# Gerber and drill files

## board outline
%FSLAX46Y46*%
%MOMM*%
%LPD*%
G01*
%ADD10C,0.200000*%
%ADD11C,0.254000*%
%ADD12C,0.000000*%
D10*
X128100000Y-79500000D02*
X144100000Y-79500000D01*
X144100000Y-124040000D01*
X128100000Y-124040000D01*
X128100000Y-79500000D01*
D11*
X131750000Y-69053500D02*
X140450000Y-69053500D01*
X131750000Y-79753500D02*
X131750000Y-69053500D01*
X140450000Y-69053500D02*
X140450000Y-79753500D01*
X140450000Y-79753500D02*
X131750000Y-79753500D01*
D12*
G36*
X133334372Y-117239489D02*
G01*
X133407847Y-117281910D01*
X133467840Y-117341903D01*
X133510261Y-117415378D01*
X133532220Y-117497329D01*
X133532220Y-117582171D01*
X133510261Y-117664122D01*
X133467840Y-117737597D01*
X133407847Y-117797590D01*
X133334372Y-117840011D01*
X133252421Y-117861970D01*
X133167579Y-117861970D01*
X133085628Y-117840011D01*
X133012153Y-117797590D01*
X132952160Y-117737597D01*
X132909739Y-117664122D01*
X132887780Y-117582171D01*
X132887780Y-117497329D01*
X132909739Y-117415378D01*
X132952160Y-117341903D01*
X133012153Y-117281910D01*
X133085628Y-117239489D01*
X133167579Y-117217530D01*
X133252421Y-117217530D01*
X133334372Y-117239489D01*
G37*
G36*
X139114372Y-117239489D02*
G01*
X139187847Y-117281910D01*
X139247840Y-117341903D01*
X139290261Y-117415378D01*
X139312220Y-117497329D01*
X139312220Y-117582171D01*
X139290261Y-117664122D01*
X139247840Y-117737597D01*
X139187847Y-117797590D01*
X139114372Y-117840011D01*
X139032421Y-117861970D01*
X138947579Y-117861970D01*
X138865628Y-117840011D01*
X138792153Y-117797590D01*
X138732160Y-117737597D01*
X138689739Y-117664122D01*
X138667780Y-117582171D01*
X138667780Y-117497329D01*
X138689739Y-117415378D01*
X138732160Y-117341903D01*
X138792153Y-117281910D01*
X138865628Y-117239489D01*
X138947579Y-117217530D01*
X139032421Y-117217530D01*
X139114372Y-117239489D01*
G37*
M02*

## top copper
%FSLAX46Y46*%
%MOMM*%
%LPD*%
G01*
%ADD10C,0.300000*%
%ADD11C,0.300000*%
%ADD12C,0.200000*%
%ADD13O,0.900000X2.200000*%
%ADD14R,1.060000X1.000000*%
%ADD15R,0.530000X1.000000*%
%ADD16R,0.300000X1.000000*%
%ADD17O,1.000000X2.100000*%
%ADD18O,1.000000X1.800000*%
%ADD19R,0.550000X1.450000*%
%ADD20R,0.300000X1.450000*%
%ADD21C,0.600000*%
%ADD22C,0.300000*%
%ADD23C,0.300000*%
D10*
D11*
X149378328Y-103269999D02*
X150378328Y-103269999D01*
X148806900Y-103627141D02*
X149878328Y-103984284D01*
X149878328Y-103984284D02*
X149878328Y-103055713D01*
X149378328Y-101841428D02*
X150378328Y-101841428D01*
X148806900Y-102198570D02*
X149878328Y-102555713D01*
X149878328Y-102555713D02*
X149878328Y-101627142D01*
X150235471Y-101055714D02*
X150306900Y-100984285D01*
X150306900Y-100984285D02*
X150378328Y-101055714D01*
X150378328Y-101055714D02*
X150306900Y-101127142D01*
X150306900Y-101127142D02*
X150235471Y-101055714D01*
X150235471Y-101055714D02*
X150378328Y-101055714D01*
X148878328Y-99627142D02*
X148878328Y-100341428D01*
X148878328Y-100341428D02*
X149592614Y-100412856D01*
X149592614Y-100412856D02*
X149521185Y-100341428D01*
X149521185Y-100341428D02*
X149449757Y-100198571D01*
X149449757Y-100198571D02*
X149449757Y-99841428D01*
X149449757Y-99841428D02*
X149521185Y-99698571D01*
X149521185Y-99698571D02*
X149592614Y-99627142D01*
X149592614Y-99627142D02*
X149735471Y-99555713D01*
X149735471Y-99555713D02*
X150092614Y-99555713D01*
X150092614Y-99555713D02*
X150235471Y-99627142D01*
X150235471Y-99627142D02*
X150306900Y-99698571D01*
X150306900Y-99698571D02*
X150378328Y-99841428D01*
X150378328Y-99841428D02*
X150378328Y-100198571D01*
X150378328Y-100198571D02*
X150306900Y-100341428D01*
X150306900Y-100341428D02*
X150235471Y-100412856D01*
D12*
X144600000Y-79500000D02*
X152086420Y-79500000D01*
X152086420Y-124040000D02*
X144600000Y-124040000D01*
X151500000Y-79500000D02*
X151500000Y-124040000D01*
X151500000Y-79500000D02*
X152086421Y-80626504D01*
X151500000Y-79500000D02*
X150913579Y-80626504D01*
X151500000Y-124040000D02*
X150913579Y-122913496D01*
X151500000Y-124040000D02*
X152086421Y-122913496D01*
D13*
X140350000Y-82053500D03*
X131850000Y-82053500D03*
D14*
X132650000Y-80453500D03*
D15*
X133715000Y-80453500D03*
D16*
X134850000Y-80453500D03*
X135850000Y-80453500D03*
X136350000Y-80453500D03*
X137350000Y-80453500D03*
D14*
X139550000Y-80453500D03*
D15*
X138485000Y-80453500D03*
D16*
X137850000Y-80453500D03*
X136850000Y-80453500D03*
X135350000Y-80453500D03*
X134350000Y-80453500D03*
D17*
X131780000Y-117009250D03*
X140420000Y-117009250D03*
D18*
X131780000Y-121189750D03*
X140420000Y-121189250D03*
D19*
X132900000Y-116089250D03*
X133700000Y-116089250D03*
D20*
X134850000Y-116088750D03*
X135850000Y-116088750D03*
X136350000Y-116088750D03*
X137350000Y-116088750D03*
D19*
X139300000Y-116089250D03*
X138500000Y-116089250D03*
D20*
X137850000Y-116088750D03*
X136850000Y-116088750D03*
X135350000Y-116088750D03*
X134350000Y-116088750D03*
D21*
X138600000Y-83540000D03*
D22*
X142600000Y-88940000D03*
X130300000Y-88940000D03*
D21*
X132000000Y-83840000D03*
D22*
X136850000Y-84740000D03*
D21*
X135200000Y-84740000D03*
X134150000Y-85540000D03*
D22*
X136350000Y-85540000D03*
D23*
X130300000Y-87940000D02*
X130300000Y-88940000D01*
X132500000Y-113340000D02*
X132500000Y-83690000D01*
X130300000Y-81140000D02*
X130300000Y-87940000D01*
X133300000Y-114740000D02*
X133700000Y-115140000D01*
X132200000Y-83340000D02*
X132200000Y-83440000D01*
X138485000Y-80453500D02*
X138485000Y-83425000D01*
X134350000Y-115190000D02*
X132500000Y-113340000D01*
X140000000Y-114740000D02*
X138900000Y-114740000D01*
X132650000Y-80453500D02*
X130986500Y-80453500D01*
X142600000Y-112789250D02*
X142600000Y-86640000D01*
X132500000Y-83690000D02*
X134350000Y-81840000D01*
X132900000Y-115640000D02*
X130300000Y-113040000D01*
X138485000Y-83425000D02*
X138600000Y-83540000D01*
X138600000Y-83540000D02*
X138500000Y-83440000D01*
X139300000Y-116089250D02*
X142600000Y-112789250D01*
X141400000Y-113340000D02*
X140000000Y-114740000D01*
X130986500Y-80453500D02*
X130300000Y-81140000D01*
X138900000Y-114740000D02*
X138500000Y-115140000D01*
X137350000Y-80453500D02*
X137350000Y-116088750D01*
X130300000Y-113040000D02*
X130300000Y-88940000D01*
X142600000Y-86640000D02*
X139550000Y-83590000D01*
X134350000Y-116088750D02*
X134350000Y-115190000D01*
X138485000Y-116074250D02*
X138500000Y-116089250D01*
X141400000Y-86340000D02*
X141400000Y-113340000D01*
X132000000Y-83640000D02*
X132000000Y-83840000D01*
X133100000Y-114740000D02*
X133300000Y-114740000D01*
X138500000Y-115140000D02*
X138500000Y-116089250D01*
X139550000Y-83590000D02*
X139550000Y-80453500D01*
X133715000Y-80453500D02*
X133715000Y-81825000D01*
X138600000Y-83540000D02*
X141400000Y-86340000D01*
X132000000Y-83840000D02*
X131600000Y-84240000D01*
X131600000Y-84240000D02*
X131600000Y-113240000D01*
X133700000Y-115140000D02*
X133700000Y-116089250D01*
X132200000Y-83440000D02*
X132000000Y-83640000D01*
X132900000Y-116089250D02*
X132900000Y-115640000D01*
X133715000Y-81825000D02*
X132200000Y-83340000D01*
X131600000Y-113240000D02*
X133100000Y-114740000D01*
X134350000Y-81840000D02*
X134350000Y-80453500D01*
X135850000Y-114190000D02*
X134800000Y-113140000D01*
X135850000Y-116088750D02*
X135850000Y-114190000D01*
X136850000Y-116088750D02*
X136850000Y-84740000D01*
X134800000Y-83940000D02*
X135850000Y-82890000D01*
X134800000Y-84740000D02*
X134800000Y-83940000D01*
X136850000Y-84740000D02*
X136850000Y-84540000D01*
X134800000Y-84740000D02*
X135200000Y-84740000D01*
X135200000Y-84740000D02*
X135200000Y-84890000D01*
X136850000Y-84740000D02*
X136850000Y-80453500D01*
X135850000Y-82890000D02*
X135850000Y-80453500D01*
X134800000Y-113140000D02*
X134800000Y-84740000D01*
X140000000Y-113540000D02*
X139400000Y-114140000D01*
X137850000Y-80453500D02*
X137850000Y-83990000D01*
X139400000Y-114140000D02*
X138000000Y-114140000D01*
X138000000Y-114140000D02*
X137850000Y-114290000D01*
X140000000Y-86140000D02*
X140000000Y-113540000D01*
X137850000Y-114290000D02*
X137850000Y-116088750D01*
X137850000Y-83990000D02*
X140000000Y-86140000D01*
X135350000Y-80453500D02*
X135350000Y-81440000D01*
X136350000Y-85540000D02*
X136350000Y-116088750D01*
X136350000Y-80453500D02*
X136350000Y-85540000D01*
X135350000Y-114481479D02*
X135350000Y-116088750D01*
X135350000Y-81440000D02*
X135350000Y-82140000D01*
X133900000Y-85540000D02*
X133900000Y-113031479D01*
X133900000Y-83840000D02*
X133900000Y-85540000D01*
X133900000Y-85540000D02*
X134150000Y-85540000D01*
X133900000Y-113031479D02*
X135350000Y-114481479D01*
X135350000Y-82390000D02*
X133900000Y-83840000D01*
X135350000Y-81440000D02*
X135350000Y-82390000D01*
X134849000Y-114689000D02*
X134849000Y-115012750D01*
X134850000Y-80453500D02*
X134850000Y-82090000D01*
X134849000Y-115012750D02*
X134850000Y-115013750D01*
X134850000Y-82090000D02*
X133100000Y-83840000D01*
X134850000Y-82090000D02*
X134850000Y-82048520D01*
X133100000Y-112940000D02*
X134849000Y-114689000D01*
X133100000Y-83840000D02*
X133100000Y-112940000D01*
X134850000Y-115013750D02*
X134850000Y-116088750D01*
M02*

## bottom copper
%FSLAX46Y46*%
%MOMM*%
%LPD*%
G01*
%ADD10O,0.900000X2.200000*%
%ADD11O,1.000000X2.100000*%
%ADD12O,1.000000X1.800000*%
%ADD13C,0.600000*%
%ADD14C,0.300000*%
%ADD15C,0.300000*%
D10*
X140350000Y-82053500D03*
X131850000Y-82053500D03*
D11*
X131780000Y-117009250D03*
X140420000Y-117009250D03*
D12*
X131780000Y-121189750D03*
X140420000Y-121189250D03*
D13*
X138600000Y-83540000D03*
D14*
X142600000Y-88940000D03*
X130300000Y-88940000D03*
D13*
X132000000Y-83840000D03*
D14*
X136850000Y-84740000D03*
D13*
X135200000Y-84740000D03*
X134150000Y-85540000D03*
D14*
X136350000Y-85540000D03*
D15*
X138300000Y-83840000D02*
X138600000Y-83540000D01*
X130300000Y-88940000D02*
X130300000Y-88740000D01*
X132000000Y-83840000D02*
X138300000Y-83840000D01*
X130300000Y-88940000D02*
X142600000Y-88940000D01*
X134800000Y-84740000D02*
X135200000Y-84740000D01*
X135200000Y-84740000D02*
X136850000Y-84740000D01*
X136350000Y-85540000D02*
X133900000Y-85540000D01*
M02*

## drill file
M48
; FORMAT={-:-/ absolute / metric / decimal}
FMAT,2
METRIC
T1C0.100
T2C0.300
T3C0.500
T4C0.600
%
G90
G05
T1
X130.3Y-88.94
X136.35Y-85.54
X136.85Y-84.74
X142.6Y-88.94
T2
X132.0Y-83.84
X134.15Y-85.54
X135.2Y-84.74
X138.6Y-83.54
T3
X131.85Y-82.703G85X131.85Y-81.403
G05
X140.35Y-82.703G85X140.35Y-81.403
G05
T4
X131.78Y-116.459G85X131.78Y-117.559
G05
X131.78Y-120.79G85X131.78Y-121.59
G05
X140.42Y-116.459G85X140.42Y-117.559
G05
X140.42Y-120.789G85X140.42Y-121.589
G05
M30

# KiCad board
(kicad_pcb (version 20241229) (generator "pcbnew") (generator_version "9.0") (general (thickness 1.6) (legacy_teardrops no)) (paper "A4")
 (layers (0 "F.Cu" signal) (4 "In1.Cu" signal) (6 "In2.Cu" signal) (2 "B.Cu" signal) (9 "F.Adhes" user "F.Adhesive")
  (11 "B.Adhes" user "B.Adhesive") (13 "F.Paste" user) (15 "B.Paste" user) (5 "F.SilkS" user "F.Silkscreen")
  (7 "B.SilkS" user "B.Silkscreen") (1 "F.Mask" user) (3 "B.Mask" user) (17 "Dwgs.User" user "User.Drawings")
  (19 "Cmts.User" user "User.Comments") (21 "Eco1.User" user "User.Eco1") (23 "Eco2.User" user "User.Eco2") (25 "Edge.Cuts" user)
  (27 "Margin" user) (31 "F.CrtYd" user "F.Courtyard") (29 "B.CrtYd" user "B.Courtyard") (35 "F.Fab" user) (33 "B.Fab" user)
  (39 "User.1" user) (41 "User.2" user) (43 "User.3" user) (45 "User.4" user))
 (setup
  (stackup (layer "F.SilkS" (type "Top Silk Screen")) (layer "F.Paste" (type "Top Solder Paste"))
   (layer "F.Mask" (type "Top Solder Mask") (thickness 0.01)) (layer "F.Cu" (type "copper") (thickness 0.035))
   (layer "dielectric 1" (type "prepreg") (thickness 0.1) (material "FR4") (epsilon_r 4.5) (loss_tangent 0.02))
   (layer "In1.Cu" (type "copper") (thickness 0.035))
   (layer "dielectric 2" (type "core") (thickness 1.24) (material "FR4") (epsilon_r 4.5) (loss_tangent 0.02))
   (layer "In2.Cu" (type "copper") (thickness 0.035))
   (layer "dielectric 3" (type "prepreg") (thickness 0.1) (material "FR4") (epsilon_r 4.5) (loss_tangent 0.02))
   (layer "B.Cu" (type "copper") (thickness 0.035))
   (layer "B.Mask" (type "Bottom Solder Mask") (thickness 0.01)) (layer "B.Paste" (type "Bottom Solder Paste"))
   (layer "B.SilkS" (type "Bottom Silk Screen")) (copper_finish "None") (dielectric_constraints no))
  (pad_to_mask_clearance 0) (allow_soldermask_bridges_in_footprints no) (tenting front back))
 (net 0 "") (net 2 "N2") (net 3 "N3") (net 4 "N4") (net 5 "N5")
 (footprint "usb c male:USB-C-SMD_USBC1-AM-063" (layer "F.Cu") (at 136.1 81.2535 180)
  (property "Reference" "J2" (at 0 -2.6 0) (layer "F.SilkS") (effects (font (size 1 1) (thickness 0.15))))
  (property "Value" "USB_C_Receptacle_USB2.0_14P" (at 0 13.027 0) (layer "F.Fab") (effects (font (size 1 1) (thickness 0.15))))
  (fp_line (start 4.35 12.2) (end -4.35 12.2) (stroke (width 0.254) (type default)) (layer "Edge.Cuts") (net 1))
  (fp_line (start 4.35 1.5) (end 4.35 12.2) (stroke (width 0.254) (type default)) (layer "Edge.Cuts") (net 1))
  (fp_line (start -4.35 12.2) (end -4.35 1.5) (stroke (width 0.254) (type default)) (layer "Edge.Cuts") (net 1))
  (fp_line (start -4.35 1.5) (end 4.35 1.5) (stroke (width 0.254) (type default)) (layer "Edge.Cuts") (net 1))
  (pad "1" thru_hole oval (at -4.25 -0.8 180) (size 0.9 2.2) (drill oval 0.5 1.8) (layers "*.Cu" "*.Mask") (remove_unused_layers no))
  (pad "2" thru_hole oval (at 4.25 -0.8 180) (size 0.9 2.2) (drill oval 0.5 1.8) (layers "*.Cu" "*.Mask") (remove_unused_layers no))
  (pad "A1B12" smd rect (at 3.45 0.8) (size 1.06 1) (layers "F.Cu" "F.Mask" "F.Paste"))
  (pad "A4B9" smd rect (at 2.385 0.8) (size 0.53 1) (layers "F.Cu" "F.Mask" "F.Paste"))
  (pad "A5" smd rect (at 1.25 0.8) (size 0.3 1) (layers "F.Cu" "F.Mask" "F.Paste") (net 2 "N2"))
  (pad "A6" smd rect (at 0.25 0.8 180) (size 0.3 1) (layers "F.Cu" "F.Mask" "F.Paste") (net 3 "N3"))
  (pad "A7" smd rect (at -0.25 0.8) (size 0.3 1) (layers "F.Cu" "F.Mask" "F.Paste") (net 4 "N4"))
  (pad "A8" smd rect (at -1.25 0.8) (size 0.3 1) (layers "F.Cu" "F.Mask" "F.Paste"))
  (pad "B1A12" smd rect (at -3.45 0.8) (size 1.06 1) (layers "F.Cu" "F.Mask" "F.Paste"))
  (pad "B4A9" smd rect (at -2.385 0.8) (size 0.53 1) (layers "F.Cu" "F.Mask" "F.Paste"))
  (pad "B5" smd rect (at -1.75 0.8) (size 0.3 1) (layers "F.Cu" "F.Mask" "F.Paste") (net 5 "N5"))
  (pad "B6" smd rect (at -0.75 0.8 180) (size 0.3 1) (layers "F.Cu" "F.Mask" "F.Paste") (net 3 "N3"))
  (pad "B7" smd rect (at 0.75 0.8) (size 0.3 1) (layers "F.Cu" "F.Mask" "F.Paste") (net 4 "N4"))
  (pad "B8" smd rect (at 1.75 0.8) (size 0.3 1) (layers "F.Cu" "F.Mask" "F.Paste")))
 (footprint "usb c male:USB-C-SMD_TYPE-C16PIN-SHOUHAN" (layer "F.Cu") (at 136.1 118.63925)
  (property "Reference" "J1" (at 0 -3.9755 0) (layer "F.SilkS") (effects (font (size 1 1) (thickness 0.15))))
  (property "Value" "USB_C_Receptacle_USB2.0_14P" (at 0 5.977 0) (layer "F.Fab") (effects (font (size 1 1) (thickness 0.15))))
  (fp_poly
   (pts (xy -2.56778 -1.141921) (xy -2.589739 -1.223872) (xy -2.63216 -1.297347) (xy -2.692153 -1.35734) (xy -2.765628 -1.399761)
    (xy -2.847579 -1.42172) (xy -2.932421 -1.42172) (xy -3.014372 -1.399761) (xy -3.087847 -1.35734) (xy -3.14784 -1.297347)
    (xy -3.190261 -1.223872) (xy -3.21222 -1.141921) (xy -3.21222 -1.057079) (xy -3.190261 -0.975128) (xy -3.14784 -0.901653)
    (xy -3.087847 -0.84166) (xy -3.014372 -0.799239) (xy -2.932421 -0.77728) (xy -2.847579 -0.77728) (xy -2.765628 -0.799239)
    (xy -2.692153 -0.84166) (xy -2.63216 -0.901653) (xy -2.589739 -0.975128) (xy -2.56778 -1.057079))
   (stroke (width 0) (type default)) (fill yes) (layer "Edge.Cuts") (net 1))
  (fp_poly
   (pts (xy 3.21222 -1.141921) (xy 3.190261 -1.223872) (xy 3.14784 -1.297347) (xy 3.087847 -1.35734) (xy 3.014372 -1.399761)
    (xy 2.932421 -1.42172) (xy 2.847579 -1.42172) (xy 2.765628 -1.399761) (xy 2.692153 -1.35734) (xy 2.63216 -1.297347)
    (xy 2.589739 -1.223872) (xy 2.56778 -1.141921) (xy 2.56778 -1.057079) (xy 2.589739 -0.975128) (xy 2.63216 -0.901653)
    (xy 2.692153 -0.84166) (xy 2.765628 -0.799239) (xy 2.847579 -0.77728) (xy 2.932421 -0.77728) (xy 3.014372 -0.799239)
    (xy 3.087847 -0.84166) (xy 3.14784 -0.901653) (xy 3.190261 -0.975128) (xy 3.21222 -1.057079))
   (stroke (width 0) (type default)) (fill yes) (layer "Edge.Cuts") (net 1))
  (pad "1" thru_hole oval (at -4.32 -1.63) (size 1 2.1) (drill oval 0.6 1.7) (layers "*.Cu" "*.Mask") (remove_unused_layers no))
  (pad "2" thru_hole oval (at 4.32 -1.63) (size 1 2.1) (drill oval 0.6 1.7) (layers "*.Cu" "*.Mask") (remove_unused_layers no))
  (pad "3" thru_hole oval (at -4.32 2.5505) (size 1 1.8) (drill oval 0.6 1.4) (layers "*.Cu" "*.Mask") (remove_unused_layers no))
  (pad "4" thru_hole oval (at 4.32 2.55) (size 1 1.8) (drill oval 0.6 1.4) (layers "*.Cu" "*.Mask") (remove_unused_layers no))
  (pad "A1B12" smd rect (at -3.2 -2.55) (size 0.55 1.45) (layers "F.Cu" "F.Mask" "F.Paste"))
  (pad "A4B9" smd rect (at -2.4 -2.55) (size 0.55 1.45) (layers "F.Cu" "F.Mask" "F.Paste"))
  (pad "A5" smd rect (at -1.25 -2.5505) (size 0.3 1.45) (layers "F.Cu" "F.Mask" "F.Paste") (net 2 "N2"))
  (pad "A6" smd rect (at -0.25 -2.5505) (size 0.3 1.45) (layers "F.Cu" "F.Mask" "F.Paste") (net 3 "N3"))
  (pad "A7" smd rect (at 0.25 -2.5505) (size 0.3 1.45) (layers "F.Cu" "F.Mask" "F.Paste") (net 4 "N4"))
  (pad "A8" smd rect (at 1.25 -2.5505) (size 0.3 1.45) (layers "F.Cu" "F.Mask" "F.Paste"))
  (pad "B1A12" smd rect (at 3.2 -2.55) (size 0.55 1.45) (layers "F.Cu" "F.Mask" "F.Paste"))
  (pad "B4A9" smd rect (at 2.4 -2.55) (size 0.55 1.45) (layers "F.Cu" "F.Mask" "F.Paste"))
  (pad "B5" smd rect (at 1.75 -2.5505) (size 0.3 1.45) (layers "F.Cu" "F.Mask" "F.Paste") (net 5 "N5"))
  (pad "B6" smd rect (at 0.75 -2.5505) (size 0.3 1.45) (layers "F.Cu" "F.Mask" "F.Paste") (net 3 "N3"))
  (pad "B7" smd rect (at -0.75 -2.5505) (size 0.3 1.45) (layers "F.Cu" "F.Mask" "F.Paste") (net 4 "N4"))
  (pad "B8" smd rect (at -1.75 -2.5505) (size 0.3 1.45) (layers "F.Cu" "F.Mask" "F.Paste")))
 (gr_rect (start 128.1 79.5) (end 144.1 124.04) (stroke (width 0.2) (type solid)) (fill no) (layer "Edge.Cuts"))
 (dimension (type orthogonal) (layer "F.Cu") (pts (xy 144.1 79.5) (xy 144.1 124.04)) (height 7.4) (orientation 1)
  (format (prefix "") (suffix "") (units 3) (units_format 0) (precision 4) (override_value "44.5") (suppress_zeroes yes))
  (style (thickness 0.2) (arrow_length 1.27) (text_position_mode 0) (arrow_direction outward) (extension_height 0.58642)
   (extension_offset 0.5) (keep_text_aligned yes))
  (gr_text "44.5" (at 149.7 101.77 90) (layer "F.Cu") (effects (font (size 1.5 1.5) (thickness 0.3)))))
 (segment (start 130.3 87.94) (end 130.3 88.94) (width 0.3) (layer "F.Cu") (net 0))
 (segment (start 132.5 113.34) (end 132.5 83.69) (width 0.3) (layer "F.Cu") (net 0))
 (segment (start 130.3 81.14) (end 130.3 87.94) (width 0.3) (layer "F.Cu") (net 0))
 (segment (start 133.3 114.74) (end 133.7 115.14) (width 0.3) (layer "F.Cu") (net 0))
 (segment (start 132.2 83.34) (end 132.2 83.44) (width 0.3) (layer "F.Cu") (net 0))
 (segment (start 138.485 80.4535) (end 138.485 83.425) (width 0.3) (layer "F.Cu") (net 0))
 (segment (start 134.35 115.19) (end 132.5 113.34) (width 0.3) (layer "F.Cu") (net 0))
 (segment (start 140 114.74) (end 138.9 114.74) (width 0.3) (layer "F.Cu") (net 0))
 (segment (start 132.65 80.4535) (end 130.9865 80.4535) (width 0.3) (layer "F.Cu") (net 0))
 (segment (start 142.6 112.78925) (end 142.6 86.64) (width 0.3) (layer "F.Cu") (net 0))
 (segment (start 132.5 83.69) (end 134.35 81.84) (width 0.3) (layer "F.Cu") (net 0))
 (segment (start 132.9 115.64) (end 130.3 113.04) (width 0.3) (layer "F.Cu") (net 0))
 (segment (start 138.485 83.425) (end 138.6 83.54) (width 0.3) (layer "F.Cu") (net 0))
 (segment (start 138.6 83.54) (end 138.5 83.44) (width 0.3) (layer "F.Cu") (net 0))
 (segment (start 139.3 116.08925) (end 142.6 112.78925) (width 0.3) (layer "F.Cu") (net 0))
 (segment (start 141.4 113.34) (end 140 114.74) (width 0.3) (layer "F.Cu") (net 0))
 (segment (start 130.9865 80.4535) (end 130.3 81.14) (width 0.3) (layer "F.Cu") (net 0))
 (segment (start 138.9 114.74) (end 138.5 115.14) (width 0.3) (layer "F.Cu") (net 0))
 (segment (start 137.35 80.4535) (end 137.35 116.08875) (width 0.3) (layer "F.Cu") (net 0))
 (segment (start 130.3 113.04) (end 130.3 88.94) (width 0.3) (layer "F.Cu") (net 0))
 (segment (start 142.6 86.64) (end 139.55 83.59) (width 0.3) (layer "F.Cu") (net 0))
 (segment (start 134.35 116.08875) (end 134.35 115.19) (width 0.3) (layer "F.Cu") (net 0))
 (segment (start 138.485 116.07425) (end 138.5 116.08925) (width 0.3) (layer "F.Cu") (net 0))
 (segment (start 141.4 86.34) (end 141.4 113.34) (width 0.3) (layer "F.Cu") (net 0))
 (segment (start 132 83.64) (end 132 83.84) (width 0.3) (layer "F.Cu") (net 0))
 (segment (start 133.1 114.74) (end 133.3 114.74) (width 0.3) (layer "F.Cu") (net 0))
 (segment (start 138.5 115.14) (end 138.5 116.08925) (width 0.3) (layer "F.Cu") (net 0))
 (segment (start 139.55 83.59) (end 139.55 80.4535) (width 0.3) (layer "F.Cu") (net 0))
 (segment (start 133.715 80.4535) (end 133.715 81.825) (width 0.3) (layer "F.Cu") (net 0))
 (segment (start 138.6 83.54) (end 141.4 86.34) (width 0.3) (layer "F.Cu") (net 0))
 (segment (start 132 83.84) (end 131.6 84.24) (width 0.3) (layer "F.Cu") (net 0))
 (segment (start 131.6 84.24) (end 131.6 113.24) (width 0.3) (layer "F.Cu") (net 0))
 (segment (start 133.7 115.14) (end 133.7 116.08925) (width 0.3) (layer "F.Cu") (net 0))
 (segment (start 132.2 83.44) (end 132 83.64) (width 0.3) (layer "F.Cu") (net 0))
 (segment (start 132.9 116.08925) (end 132.9 115.64) (width 0.3) (layer "F.Cu") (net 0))
 (segment (start 133.715 81.825) (end 132.2 83.34) (width 0.3) (layer "F.Cu") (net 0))
 (segment (start 131.6 113.24) (end 133.1 114.74) (width 0.3) (layer "F.Cu") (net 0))
 (segment (start 134.35 81.84) (end 134.35 80.4535) (width 0.3) (layer "F.Cu") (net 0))
 (via blind (at 138.6 83.54) (size 0.6) (drill 0.3) (layers "F.Cu" "B.Cu") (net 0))
 (via micro (at 142.6 88.94) (size 0.3) (drill 0.1) (layers "F.Cu" "B.Cu") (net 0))
 (via micro (at 130.3 88.94) (size 0.3) (drill 0.1) (layers "F.Cu" "B.Cu") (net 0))
 (via blind (at 132 83.84) (size 0.6) (drill 0.3) (layers "F.Cu" "B.Cu") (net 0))
 (segment (start 138.3 83.84) (end 138.6 83.54) (width 0.3) (layer "B.Cu") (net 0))
 (segment (start 130.3 88.94) (end 130.3 88.74) (width 0.3) (layer "B.Cu") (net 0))
 (segment (start 132 83.84) (end 138.3 83.84) (width 0.3) (layer "B.Cu") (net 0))
 (segment (start 130.3 88.94) (end 142.6 88.94) (width 0.3) (layer "B.Cu") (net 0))
 (segment (start 135.85 114.19) (end 134.8 113.14) (width 0.3) (layer "F.Cu") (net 3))
 (segment (start 135.85 116.08875) (end 135.85 114.19) (width 0.3) (layer "F.Cu") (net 3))
 (segment (start 136.85 116.08875) (end 136.85 84.74) (width 0.3) (layer "F.Cu") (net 3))
 (segment (start 134.8 83.94) (end 135.85 82.89) (width 0.3) (layer "F.Cu") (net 3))
 (segment (start 134.8 84.74) (end 134.8 83.94) (width 0.3) (layer "F.Cu") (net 3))
 (segment (start 136.85 84.74) (end 136.85 84.54) (width 0.3) (layer "F.Cu") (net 3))
 (segment (start 134.8 84.74) (end 135.2 84.74) (width 0.3) (layer "F.Cu") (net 3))
 (segment (start 135.2 84.74) (end 135.2 84.89) (width 0.3) (layer "F.Cu") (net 3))
 (segment (start 136.85 84.74) (end 136.85 80.4535) (width 0.3) (layer "F.Cu") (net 3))
 (segment (start 135.85 82.89) (end 135.85 80.4535) (width 0.3) (layer "F.Cu") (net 3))
 (segment (start 134.8 113.14) (end 134.8 84.74) (width 0.3) (layer "F.Cu") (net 3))
 (via micro (at 136.85 84.74) (size 0.3) (drill 0.1) (layers "F.Cu" "B.Cu") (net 3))
 (via blind (at 135.2 84.74) (size 0.6) (drill 0.3) (layers "F.Cu" "B.Cu") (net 3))
 (segment (start 134.8 84.74) (end 135.2 84.74) (width 0.3) (layer "B.Cu") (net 3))
 (segment (start 135.2 84.74) (end 136.85 84.74) (width 0.3) (layer "B.Cu") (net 3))
 (segment (start 140 113.54) (end 139.4 114.14) (width 0.3) (layer "F.Cu") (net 5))
 (segment (start 137.85 80.4535) (end 137.85 83.99) (width 0.3) (layer "F.Cu") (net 5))
 (segment (start 139.4 114.14) (end 138 114.14) (width 0.3) (layer "F.Cu") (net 5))
 (segment (start 138 114.14) (end 137.85 114.29) (width 0.3) (layer "F.Cu") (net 5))
 (segment (start 140 86.14) (end 140 113.54) (width 0.3) (layer "F.Cu") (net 5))
 (segment (start 137.85 114.29) (end 137.85 116.08875) (width 0.3) (layer "F.Cu") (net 5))
 (segment (start 137.85 83.99) (end 140 86.14) (width 0.3) (layer "F.Cu") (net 5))
 (segment (start 135.35 80.4535) (end 135.35 81.44) (width 0.3) (layer "F.Cu") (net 4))
 (segment (start 136.35 85.54) (end 136.35 116.08875) (width 0.3) (layer "F.Cu") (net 4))
 (segment (start 136.35 80.4535) (end 136.35 85.54) (width 0.3) (layer "F.Cu") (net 4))
 (segment (start 135.35 114.481479) (end 135.35 116.08875) (width 0.3) (layer "F.Cu") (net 4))
 (segment (start 135.35 81.44) (end 135.35 82.14) (width 0.3) (layer "F.Cu") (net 4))
 (segment (start 133.9 85.54) (end 133.9 113.031479) (width 0.3) (layer "F.Cu") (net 4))
 (segment (start 133.9 83.84) (end 133.9 85.54) (width 0.3) (layer "F.Cu") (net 4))
 (segment (start 133.9 85.54) (end 134.15 85.54) (width 0.3) (layer "F.Cu") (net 4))
 (segment (start 133.9 113.031479) (end 135.35 114.481479) (width 0.3) (layer "F.Cu") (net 4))
 (segment (start 135.35 82.39) (end 133.9 83.84) (width 0.3) (layer "F.Cu") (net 4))
 (segment (start 135.35 81.44) (end 135.35 82.39) (width 0.3) (layer "F.Cu") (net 4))
 (via blind (at 134.15 85.54) (size 0.6) (drill 0.3) (layers "F.Cu" "B.Cu") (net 4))
 (via micro (at 136.35 85.54) (size 0.3) (drill 0.1) (layers "F.Cu" "B.Cu") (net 4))
 (segment (start 136.35 85.54) (end 133.9 85.54) (width 0.3) (layer "B.Cu") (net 4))
 (segment (start 134.849 114.689) (end 134.849 115.01275) (width 0.3) (layer "F.Cu") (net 2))
 (segment (start 134.85 80.4535) (end 134.85 82.09) (width 0.3) (layer "F.Cu") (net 2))
 (segment (start 134.849 115.01275) (end 134.85 115.01375) (width 0.3) (layer "F.Cu") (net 2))
 (segment (start 134.85 82.09) (end 133.1 83.84) (width 0.3) (layer "F.Cu") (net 2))
 (segment (start 134.85 82.09) (end 134.85 82.04852) (width 0.3) (layer "F.Cu") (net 2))
 (segment (start 133.1 112.94) (end 134.849 114.689) (width 0.3) (layer "F.Cu") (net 2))
 (segment (start 133.1 83.84) (end 133.1 112.94) (width 0.3) (layer "F.Cu") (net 2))
 (segment (start 134.85 115.01375) (end 134.85 116.08875) (width 0.3) (layer "F.Cu") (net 2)))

